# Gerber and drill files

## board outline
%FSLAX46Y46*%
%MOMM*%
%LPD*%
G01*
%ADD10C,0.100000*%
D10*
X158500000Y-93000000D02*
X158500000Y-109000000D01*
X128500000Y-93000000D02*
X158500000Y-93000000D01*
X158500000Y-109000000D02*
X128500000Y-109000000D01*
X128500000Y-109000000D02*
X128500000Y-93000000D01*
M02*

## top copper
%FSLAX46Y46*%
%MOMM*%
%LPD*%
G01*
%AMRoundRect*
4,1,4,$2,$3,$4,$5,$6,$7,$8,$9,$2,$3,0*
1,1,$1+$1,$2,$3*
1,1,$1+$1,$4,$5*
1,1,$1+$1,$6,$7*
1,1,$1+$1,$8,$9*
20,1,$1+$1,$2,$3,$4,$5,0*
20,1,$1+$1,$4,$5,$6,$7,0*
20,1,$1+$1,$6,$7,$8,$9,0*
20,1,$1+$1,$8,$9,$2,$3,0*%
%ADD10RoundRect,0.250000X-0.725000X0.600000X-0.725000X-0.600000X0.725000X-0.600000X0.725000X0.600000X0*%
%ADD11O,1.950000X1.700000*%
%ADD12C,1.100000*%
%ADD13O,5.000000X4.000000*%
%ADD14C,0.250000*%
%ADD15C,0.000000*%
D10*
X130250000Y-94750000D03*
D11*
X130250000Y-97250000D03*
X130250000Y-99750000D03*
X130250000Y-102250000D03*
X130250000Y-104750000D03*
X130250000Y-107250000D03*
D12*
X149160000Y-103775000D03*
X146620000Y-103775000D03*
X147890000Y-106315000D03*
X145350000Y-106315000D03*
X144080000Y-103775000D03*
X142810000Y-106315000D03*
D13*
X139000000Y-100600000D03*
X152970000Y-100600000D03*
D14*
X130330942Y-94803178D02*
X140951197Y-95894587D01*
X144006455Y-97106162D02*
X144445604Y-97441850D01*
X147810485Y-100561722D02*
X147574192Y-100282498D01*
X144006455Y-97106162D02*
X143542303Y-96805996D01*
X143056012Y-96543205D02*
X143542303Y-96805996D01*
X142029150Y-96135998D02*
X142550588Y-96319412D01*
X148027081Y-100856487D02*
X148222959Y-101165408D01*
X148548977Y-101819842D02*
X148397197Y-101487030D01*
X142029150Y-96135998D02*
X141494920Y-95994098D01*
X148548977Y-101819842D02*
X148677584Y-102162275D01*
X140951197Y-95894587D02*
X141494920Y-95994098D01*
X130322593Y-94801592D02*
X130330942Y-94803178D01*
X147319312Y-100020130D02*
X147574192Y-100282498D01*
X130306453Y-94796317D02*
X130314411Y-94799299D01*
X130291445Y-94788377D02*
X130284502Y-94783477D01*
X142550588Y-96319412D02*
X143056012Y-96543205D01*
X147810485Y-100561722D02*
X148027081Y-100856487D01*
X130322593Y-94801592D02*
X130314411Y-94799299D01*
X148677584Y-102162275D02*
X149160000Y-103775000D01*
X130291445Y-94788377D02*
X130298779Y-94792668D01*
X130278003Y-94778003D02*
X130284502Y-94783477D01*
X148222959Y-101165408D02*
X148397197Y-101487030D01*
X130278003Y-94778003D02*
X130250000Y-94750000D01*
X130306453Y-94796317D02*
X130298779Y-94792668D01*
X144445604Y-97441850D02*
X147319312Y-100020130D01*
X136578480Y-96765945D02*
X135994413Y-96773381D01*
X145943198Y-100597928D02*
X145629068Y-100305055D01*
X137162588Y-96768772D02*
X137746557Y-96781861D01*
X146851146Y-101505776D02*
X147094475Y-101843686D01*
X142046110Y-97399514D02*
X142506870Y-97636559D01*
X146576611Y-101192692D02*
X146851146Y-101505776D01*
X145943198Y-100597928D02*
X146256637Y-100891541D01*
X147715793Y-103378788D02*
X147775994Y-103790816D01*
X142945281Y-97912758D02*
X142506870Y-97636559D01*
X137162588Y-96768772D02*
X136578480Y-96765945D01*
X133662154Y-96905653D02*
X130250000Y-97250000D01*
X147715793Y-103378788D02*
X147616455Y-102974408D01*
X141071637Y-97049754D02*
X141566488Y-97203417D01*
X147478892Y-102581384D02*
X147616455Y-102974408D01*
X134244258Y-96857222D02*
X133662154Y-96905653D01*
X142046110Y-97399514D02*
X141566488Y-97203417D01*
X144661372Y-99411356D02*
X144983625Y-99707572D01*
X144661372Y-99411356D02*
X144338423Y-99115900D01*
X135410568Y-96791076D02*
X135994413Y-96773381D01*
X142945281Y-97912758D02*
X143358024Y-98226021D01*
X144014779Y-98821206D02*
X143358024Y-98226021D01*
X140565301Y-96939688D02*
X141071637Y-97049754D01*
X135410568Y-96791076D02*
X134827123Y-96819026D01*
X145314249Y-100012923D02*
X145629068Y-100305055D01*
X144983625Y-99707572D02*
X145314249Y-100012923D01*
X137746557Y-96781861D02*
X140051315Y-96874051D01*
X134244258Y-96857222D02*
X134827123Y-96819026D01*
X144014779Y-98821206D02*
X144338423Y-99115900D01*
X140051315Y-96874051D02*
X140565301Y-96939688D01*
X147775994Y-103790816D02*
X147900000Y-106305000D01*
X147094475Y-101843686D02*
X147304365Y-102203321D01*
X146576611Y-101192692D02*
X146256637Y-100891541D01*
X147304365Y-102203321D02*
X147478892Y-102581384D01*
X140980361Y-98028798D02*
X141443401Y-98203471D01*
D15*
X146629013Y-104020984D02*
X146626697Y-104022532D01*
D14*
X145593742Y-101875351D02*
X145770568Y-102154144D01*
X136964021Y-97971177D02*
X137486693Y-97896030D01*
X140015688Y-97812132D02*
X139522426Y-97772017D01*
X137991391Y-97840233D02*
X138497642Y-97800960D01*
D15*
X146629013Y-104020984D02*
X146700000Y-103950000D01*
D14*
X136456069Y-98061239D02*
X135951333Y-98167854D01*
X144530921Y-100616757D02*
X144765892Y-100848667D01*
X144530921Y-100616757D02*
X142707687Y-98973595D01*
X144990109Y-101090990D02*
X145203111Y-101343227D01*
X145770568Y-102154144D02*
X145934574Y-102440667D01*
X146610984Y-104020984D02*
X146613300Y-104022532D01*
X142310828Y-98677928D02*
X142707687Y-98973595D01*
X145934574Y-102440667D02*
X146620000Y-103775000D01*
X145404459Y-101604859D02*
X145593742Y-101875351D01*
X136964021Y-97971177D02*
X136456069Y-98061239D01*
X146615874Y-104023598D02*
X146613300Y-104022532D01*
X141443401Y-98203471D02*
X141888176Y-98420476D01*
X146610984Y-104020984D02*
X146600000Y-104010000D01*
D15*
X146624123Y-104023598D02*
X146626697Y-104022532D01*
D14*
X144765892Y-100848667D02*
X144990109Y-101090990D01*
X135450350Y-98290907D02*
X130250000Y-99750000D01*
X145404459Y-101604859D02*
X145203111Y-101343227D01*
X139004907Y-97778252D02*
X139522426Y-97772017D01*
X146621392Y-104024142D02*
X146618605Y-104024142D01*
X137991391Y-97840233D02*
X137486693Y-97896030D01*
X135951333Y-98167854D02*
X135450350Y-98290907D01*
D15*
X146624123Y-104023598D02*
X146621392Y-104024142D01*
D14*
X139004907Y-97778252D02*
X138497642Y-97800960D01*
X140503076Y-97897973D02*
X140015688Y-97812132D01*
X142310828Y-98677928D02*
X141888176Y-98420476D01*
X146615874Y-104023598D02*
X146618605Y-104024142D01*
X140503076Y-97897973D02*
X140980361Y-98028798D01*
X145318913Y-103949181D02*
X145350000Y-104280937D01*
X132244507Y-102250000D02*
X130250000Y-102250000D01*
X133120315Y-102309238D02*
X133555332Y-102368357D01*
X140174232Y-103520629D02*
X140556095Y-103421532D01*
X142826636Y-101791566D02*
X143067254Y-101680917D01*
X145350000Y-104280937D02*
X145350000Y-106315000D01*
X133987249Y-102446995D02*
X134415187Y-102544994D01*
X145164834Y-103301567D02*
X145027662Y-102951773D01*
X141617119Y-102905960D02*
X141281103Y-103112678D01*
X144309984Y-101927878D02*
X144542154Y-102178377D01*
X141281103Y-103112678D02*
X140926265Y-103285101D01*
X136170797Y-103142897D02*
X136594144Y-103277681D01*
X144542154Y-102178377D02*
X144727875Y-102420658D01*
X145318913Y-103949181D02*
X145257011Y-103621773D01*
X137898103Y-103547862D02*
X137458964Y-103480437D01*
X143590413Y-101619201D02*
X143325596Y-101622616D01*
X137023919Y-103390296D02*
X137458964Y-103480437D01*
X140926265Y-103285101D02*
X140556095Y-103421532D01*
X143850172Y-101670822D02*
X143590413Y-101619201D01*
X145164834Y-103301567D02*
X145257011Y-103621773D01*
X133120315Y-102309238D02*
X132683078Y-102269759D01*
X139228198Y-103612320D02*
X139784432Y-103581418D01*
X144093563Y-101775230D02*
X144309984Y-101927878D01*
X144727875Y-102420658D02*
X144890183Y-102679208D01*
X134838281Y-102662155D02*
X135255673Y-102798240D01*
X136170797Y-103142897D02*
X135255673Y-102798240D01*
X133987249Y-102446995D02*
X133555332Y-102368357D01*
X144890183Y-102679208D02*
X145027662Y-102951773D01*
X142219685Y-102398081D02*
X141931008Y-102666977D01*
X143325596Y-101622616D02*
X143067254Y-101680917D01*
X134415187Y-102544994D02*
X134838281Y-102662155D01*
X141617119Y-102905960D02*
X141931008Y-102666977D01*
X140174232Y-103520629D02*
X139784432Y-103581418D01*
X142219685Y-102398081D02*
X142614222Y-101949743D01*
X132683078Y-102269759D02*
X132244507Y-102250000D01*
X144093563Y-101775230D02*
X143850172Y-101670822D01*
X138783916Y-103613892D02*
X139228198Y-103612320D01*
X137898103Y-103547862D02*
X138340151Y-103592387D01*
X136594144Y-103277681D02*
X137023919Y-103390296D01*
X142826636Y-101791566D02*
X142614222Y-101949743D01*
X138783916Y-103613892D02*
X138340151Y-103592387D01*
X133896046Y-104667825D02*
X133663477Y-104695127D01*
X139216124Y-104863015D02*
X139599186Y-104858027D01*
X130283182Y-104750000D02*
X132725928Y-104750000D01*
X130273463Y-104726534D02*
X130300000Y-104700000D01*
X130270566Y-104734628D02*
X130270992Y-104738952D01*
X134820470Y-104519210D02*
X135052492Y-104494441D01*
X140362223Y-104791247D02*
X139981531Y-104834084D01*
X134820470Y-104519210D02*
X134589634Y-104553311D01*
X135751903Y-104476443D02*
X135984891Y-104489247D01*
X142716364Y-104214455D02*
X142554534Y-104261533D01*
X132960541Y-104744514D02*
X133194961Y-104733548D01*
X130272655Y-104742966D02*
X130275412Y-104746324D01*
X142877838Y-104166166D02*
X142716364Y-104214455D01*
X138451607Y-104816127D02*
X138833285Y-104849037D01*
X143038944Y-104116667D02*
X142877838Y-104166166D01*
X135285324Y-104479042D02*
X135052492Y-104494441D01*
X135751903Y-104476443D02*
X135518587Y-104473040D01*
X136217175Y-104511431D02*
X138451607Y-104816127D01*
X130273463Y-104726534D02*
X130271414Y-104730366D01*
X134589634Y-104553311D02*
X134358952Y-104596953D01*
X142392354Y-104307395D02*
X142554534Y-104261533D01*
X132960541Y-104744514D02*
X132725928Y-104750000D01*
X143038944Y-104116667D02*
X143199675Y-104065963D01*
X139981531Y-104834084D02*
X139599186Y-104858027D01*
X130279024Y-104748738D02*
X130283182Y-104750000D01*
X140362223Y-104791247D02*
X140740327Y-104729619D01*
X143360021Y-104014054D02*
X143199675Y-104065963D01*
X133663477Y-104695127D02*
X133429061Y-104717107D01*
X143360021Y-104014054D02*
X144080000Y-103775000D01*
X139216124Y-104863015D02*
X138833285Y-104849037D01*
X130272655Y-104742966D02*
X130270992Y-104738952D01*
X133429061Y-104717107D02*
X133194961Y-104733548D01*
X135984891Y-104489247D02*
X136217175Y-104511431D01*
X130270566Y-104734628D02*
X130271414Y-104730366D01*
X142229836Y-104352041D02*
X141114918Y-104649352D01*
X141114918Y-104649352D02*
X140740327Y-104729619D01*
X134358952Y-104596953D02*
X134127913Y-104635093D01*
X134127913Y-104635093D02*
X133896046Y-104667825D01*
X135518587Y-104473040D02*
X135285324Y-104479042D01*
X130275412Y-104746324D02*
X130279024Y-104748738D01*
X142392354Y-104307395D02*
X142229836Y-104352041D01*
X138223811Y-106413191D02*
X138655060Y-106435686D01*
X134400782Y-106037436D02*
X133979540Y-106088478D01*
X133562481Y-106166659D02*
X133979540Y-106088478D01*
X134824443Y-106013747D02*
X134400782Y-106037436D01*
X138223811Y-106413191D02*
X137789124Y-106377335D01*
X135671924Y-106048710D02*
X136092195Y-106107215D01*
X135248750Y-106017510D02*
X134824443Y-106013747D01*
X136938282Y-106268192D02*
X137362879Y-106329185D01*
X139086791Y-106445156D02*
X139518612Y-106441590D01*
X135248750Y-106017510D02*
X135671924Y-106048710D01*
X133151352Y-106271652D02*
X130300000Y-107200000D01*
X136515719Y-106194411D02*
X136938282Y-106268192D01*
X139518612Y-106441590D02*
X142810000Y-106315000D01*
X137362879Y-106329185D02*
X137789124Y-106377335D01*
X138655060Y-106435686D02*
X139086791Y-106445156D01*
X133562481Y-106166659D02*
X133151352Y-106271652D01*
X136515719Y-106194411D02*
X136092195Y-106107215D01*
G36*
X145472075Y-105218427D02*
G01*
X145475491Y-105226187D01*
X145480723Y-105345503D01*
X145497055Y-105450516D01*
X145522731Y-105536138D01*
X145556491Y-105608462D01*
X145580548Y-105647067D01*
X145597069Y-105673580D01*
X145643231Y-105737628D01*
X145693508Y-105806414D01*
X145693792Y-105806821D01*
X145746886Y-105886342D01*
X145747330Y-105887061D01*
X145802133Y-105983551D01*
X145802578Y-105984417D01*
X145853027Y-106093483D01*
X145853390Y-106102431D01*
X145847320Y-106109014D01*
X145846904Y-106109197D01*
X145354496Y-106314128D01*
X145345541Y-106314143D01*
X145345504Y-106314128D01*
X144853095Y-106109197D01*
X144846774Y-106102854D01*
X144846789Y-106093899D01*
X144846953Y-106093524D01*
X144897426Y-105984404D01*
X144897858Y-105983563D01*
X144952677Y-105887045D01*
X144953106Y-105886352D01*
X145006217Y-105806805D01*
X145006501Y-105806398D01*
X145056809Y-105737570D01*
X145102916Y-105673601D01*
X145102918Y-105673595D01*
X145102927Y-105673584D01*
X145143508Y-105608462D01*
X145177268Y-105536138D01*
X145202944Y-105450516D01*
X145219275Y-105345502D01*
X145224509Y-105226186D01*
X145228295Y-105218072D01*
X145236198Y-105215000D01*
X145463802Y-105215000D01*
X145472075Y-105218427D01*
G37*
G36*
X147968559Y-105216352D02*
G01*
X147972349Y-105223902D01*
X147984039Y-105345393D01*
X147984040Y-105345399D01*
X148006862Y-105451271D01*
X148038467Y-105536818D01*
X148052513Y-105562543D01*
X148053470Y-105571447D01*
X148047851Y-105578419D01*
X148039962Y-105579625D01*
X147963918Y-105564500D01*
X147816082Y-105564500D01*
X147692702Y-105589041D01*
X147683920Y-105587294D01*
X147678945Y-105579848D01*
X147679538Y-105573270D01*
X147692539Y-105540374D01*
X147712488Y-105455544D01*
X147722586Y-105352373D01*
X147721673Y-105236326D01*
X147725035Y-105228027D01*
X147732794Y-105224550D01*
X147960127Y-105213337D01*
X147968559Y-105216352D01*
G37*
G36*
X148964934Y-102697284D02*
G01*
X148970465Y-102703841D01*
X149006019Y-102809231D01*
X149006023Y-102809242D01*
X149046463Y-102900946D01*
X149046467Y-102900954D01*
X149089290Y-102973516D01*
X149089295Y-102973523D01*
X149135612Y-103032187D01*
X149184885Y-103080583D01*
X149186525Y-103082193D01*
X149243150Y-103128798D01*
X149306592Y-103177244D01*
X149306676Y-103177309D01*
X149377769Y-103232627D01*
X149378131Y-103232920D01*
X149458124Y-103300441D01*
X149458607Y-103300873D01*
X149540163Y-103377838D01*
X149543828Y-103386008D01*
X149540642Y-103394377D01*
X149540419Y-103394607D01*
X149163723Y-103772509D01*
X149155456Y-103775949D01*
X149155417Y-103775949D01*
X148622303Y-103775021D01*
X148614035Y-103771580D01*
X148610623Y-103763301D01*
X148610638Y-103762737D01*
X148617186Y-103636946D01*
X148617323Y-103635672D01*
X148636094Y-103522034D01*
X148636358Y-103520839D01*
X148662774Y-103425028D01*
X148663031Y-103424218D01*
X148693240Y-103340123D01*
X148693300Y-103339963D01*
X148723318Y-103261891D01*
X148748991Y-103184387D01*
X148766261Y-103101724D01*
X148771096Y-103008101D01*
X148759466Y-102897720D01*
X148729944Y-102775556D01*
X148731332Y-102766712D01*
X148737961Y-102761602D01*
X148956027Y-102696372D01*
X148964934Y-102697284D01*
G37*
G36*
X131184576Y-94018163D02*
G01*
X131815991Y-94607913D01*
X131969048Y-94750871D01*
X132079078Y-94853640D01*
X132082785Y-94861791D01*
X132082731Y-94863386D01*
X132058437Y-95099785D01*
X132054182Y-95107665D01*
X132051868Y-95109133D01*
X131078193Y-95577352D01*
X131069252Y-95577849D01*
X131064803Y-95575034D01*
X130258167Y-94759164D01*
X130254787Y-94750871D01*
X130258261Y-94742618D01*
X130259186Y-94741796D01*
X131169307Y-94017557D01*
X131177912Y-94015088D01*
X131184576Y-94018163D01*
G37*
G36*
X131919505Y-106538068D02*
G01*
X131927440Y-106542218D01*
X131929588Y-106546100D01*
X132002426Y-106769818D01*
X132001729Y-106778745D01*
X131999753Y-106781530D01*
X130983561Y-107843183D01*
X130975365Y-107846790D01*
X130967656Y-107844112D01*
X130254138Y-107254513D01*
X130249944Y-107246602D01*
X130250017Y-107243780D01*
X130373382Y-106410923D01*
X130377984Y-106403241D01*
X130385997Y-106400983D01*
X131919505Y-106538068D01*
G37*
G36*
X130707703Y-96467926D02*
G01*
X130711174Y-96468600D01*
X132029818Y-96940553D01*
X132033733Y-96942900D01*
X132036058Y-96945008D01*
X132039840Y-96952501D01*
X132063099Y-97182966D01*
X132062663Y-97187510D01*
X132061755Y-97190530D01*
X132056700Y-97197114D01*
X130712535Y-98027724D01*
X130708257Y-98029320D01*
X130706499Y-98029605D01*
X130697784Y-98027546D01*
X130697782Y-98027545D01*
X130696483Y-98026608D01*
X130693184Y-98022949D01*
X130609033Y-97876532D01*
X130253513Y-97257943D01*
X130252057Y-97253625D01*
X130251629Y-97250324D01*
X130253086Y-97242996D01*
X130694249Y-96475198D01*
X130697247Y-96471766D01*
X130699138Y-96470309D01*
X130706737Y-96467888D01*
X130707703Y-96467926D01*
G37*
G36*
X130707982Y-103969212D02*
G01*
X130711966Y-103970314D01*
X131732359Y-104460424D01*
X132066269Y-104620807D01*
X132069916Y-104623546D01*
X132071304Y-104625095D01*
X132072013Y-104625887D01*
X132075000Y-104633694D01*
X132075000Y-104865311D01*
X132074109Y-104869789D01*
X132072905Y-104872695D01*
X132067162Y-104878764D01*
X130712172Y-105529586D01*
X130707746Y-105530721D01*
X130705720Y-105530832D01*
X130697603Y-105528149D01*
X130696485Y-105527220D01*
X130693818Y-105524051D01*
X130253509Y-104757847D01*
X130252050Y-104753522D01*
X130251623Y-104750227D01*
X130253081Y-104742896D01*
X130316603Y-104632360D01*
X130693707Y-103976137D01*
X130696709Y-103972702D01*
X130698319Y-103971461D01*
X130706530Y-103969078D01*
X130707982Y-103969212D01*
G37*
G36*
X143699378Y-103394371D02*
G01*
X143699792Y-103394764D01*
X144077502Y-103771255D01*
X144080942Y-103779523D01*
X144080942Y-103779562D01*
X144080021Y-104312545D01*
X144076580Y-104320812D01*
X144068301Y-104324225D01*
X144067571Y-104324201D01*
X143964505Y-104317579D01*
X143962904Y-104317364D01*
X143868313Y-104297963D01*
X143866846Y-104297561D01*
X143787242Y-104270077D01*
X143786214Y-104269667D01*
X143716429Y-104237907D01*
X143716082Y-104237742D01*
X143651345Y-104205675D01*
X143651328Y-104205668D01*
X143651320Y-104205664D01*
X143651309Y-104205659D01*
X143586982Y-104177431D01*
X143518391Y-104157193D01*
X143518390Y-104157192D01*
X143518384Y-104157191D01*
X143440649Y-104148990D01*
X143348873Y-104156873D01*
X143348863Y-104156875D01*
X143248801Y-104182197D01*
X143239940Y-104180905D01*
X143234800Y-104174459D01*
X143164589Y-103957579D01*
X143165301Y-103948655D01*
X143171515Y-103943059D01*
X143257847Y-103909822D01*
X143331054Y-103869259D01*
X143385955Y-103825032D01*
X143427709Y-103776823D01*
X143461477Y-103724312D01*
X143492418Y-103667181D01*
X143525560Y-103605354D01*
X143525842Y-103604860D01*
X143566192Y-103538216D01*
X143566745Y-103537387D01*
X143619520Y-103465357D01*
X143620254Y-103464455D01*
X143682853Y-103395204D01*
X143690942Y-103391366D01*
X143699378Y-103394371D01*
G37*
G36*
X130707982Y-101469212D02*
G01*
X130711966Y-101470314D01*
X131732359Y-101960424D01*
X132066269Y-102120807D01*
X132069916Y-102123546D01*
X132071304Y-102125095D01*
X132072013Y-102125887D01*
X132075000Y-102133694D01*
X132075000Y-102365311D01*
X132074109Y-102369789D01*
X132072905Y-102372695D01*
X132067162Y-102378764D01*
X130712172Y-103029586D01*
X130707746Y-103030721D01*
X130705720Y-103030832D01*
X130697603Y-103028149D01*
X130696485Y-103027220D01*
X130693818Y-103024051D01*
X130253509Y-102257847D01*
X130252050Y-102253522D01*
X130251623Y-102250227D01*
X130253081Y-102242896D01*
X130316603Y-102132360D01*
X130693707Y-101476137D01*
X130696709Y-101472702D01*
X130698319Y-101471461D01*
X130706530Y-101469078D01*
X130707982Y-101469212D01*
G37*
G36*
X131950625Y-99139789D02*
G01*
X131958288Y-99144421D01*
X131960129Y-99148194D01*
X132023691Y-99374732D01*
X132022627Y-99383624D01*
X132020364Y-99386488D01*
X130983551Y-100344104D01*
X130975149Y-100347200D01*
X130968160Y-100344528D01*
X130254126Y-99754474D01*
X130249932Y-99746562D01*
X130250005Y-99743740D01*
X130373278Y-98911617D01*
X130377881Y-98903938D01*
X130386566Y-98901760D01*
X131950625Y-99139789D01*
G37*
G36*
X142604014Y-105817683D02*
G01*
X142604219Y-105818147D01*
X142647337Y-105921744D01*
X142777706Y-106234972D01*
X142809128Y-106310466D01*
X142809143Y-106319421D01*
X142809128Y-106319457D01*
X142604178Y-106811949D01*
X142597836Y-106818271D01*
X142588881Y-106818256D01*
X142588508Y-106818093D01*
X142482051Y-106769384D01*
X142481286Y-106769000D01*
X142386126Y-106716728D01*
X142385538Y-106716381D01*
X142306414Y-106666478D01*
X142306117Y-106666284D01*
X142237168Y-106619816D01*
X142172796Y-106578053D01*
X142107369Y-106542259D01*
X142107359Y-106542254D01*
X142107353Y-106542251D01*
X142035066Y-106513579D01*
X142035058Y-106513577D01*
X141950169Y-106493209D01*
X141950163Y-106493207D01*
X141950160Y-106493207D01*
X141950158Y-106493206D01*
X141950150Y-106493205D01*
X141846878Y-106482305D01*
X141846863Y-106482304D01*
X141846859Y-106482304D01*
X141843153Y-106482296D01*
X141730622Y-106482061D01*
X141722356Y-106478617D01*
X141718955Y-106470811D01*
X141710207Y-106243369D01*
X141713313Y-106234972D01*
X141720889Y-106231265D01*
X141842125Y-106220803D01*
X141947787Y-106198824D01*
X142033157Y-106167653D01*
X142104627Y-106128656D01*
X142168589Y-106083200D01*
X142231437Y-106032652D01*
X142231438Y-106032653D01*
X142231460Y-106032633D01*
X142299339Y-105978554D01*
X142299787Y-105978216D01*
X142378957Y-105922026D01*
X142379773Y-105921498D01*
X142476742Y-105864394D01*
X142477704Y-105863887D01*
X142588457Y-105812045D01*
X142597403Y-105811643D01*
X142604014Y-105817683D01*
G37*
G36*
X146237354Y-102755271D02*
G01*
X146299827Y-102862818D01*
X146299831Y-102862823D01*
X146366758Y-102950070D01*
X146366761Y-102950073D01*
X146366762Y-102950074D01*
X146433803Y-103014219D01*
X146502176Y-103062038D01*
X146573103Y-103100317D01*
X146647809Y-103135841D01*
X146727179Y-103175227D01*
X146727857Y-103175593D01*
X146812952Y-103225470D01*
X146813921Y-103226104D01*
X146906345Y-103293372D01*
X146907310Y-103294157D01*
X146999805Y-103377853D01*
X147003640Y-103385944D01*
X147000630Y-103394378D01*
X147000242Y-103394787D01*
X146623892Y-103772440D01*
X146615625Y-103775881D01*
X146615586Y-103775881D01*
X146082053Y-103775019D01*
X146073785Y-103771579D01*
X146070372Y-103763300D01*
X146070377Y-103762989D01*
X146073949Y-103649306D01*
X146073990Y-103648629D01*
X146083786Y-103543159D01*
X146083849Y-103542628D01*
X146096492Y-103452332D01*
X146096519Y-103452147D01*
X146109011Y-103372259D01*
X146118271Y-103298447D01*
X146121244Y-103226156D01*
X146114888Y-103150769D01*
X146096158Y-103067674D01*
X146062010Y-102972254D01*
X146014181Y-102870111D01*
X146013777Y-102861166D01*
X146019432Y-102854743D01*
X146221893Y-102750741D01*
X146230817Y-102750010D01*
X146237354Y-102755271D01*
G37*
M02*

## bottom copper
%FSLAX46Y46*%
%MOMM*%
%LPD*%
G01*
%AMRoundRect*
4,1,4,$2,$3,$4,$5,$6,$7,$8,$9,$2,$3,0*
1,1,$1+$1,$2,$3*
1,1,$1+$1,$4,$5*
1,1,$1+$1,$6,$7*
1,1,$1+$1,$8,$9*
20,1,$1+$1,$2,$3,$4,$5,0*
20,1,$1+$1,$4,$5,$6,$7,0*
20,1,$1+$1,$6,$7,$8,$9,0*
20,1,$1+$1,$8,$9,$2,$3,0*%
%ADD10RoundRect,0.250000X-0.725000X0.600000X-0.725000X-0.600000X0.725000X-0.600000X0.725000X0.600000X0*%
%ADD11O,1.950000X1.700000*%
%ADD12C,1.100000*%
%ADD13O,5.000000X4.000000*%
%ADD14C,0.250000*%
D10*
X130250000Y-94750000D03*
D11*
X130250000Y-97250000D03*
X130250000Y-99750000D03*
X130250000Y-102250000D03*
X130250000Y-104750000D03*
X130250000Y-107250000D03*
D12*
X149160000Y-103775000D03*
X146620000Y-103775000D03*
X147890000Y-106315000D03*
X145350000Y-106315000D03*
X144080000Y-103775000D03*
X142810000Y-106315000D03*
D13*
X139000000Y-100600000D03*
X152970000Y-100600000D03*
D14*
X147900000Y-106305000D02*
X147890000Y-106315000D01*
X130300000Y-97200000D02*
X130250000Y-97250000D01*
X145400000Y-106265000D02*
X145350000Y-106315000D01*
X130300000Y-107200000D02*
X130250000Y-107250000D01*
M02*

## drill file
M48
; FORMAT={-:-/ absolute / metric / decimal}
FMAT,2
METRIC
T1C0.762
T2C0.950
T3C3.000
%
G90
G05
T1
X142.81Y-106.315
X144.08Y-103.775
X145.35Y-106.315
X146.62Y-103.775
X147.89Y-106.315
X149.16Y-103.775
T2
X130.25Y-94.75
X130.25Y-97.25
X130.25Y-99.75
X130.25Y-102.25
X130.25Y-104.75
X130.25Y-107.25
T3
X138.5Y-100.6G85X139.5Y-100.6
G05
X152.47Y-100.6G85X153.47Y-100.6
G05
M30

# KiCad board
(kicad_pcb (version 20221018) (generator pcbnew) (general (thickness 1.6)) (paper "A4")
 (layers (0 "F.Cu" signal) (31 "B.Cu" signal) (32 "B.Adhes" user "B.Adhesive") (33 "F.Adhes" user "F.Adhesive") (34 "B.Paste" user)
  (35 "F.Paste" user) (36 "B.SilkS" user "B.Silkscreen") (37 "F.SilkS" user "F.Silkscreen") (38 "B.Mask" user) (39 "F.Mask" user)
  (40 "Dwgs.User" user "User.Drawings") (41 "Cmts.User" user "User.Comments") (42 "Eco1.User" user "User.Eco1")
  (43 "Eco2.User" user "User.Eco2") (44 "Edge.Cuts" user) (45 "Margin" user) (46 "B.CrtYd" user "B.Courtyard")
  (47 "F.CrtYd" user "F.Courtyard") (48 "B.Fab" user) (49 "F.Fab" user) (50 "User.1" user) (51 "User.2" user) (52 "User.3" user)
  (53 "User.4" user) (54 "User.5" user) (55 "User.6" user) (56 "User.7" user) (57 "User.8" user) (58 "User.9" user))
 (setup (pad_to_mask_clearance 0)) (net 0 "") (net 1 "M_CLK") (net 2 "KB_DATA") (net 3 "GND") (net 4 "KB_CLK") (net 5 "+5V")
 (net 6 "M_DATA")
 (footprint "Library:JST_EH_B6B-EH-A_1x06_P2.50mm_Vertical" (layer "F.Cu") (at 130.25 94.75 -90)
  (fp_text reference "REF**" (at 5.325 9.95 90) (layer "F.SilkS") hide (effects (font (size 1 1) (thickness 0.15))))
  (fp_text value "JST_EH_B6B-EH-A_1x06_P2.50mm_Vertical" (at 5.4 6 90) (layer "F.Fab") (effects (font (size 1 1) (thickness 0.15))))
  (pad "1" thru_hole roundrect (at 0 0 270) (size 1.7 1.95) (drill 0.95) (layers "*.Cu" "*.Mask") (roundrect_rratio 0.1470588235)
   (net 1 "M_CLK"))
  (pad "2" thru_hole oval (at 2.5 0 270) (size 1.7 1.95) (drill 0.95) (layers "*.Cu" "*.Mask") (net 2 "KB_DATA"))
  (pad "3" thru_hole oval (at 5 0 270) (size 1.7 1.95) (drill 0.95) (layers "*.Cu" "*.Mask") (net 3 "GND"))
  (pad "4" thru_hole oval (at 7.5 0 270) (size 1.7 1.95) (drill 0.95) (layers "*.Cu" "*.Mask") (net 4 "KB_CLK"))
  (pad "5" thru_hole oval (at 10 0 270) (size 1.7 1.95) (drill 0.95) (layers "*.Cu" "*.Mask") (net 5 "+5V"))
  (pad "6" thru_hole oval (at 12.5 0 270) (size 1.7 1.95) (drill 0.95) (layers "*.Cu" "*.Mask") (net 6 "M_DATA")))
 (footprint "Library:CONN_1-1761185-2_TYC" (layer "F.Cu") (at 142.81 106.315)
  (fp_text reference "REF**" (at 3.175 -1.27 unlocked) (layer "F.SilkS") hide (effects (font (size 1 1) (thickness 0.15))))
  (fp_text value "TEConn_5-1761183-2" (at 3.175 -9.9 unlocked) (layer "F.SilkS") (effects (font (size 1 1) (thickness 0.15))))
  (pad "1" thru_hole circle (at 6.35 -2.54) (size 1.1 1.1) (drill 0.762) (layers "*.Cu" "*.Mask") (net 1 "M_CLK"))
  (pad "3" thru_hole circle (at 3.81 -2.54) (size 1.1 1.1) (drill 0.762) (layers "*.Cu" "*.Mask") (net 3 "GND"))
  (pad "3" thru_hole circle (at 5.08 0) (size 1.1 1.1) (drill 0.762) (layers "*.Cu" "*.Mask") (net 3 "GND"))
  (pad "4" thru_hole circle (at 2.54 0) (size 1.1 1.1) (drill 0.762) (layers "*.Cu" "*.Mask") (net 4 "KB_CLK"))
  (pad "5" thru_hole circle (at 1.27 -2.54) (size 1.1 1.1) (drill 0.762) (layers "*.Cu" "*.Mask") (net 5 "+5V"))
  (pad "6" thru_hole circle (at 0 0) (size 1.1 1.1) (drill 0.762) (layers "*.Cu" "*.Mask") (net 6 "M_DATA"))
  (pad "13" thru_hole oval (at -3.81 -5.715) (size 5 4) (drill oval 4 3) (layers "*.Cu" "*.Mask"))
  (pad "14" thru_hole oval (at 10.16 -5.715) (size 5 4) (drill oval 4 3) (layers "*.Cu" "*.Mask")))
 (gr_line (start 158.5 93) (end 158.5 109) (stroke (width 0.1) (type default)) (layer "Edge.Cuts"))
 (gr_line (start 128.5 93) (end 158.5 93) (stroke (width 0.1) (type default)) (layer "Edge.Cuts"))
 (gr_line (start 158.5 109) (end 128.5 109) (stroke (width 0.1) (type default)) (layer "Edge.Cuts"))
 (gr_line (start 128.5 109) (end 128.5 93) (stroke (width 0.1) (type default)) (layer "Edge.Cuts"))
 (segment (start 130.330942 94.803178) (end 140.951197 95.894587) (width 0.25) (layer "F.Cu") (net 1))
 (segment (start 144.006455 97.106162) (end 144.445604 97.44185) (width 0.25) (layer "F.Cu") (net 1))
 (segment (start 147.810485 100.561722) (end 147.574192 100.282498) (width 0.25) (layer "F.Cu") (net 1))
 (segment (start 144.006455 97.106162) (end 143.542303 96.805996) (width 0.25) (layer "F.Cu") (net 1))
 (segment (start 143.056012 96.543205) (end 143.542303 96.805996) (width 0.25) (layer "F.Cu") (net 1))
 (segment (start 142.02915 96.135998) (end 142.550588 96.319412) (width 0.25) (layer "F.Cu") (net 1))
 (segment (start 148.027081 100.856487) (end 148.222959 101.165408) (width 0.25) (layer "F.Cu") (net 1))
 (segment (start 148.548977 101.819842) (end 148.397197 101.48703) (width 0.25) (layer "F.Cu") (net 1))
 (segment (start 142.02915 96.135998) (end 141.49492 95.994098) (width 0.25) (layer "F.Cu") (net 1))
 (segment (start 148.548977 101.819842) (end 148.677584 102.162275) (width 0.25) (layer "F.Cu") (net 1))
 (segment (start 140.951197 95.894587) (end 141.49492 95.994098) (width 0.25) (layer "F.Cu") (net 1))
 (segment (start 130.322593 94.801592) (end 130.330942 94.803178) (width 0.25) (layer "F.Cu") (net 1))
 (segment (start 147.319312 100.02013) (end 147.574192 100.282498) (width 0.25) (layer "F.Cu") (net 1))
 (segment (start 130.306453 94.796317) (end 130.314411 94.799299) (width 0.25) (layer "F.Cu") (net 1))
 (segment (start 130.291445 94.788377) (end 130.284502 94.783477) (width 0.25) (layer "F.Cu") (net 1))
 (segment (start 142.550588 96.319412) (end 143.056012 96.543205) (width 0.25) (layer "F.Cu") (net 1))
 (segment (start 147.810485 100.561722) (end 148.027081 100.856487) (width 0.25) (layer "F.Cu") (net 1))
 (segment (start 130.322593 94.801592) (end 130.314411 94.799299) (width 0.25) (layer "F.Cu") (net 1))
 (segment (start 148.677584 102.162275) (end 149.16 103.775) (width 0.25) (layer "F.Cu") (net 1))
 (segment (start 130.291445 94.788377) (end 130.298779 94.792668) (width 0.25) (layer "F.Cu") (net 1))
 (segment (start 130.278003 94.778003) (end 130.284502 94.783477) (width 0.25) (layer "F.Cu") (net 1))
 (segment (start 148.222959 101.165408) (end 148.397197 101.48703) (width 0.25) (layer "F.Cu") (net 1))
 (segment (start 130.278003 94.778003) (end 130.25 94.75) (width 0.25) (layer "F.Cu") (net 1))
 (segment (start 130.306453 94.796317) (end 130.298779 94.792668) (width 0.25) (layer "F.Cu") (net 1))
 (segment (start 144.445604 97.44185) (end 147.319312 100.02013) (width 0.25) (layer "F.Cu") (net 1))
 (segment (start 136.57848 96.765945) (end 135.994413 96.773381) (width 0.25) (layer "F.Cu") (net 2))
 (segment (start 145.943198 100.597928) (end 145.629068 100.305055) (width 0.25) (layer "F.Cu") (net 2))
 (segment (start 137.162588 96.768772) (end 137.746557 96.781861) (width 0.25) (layer "F.Cu") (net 2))
 (segment (start 146.851146 101.505776) (end 147.094475 101.843686) (width 0.25) (layer "F.Cu") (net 2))
 (segment (start 142.04611 97.399514) (end 142.50687 97.636559) (width 0.25) (layer "F.Cu") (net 2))
 (segment (start 146.576611 101.192692) (end 146.851146 101.505776) (width 0.25) (layer "F.Cu") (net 2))
 (segment (start 145.943198 100.597928) (end 146.256637 100.891541) (width 0.25) (layer "F.Cu") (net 2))
 (segment (start 147.715793 103.378788) (end 147.775994 103.790816) (width 0.25) (layer "F.Cu") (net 2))
 (segment (start 142.945281 97.912758) (end 142.50687 97.636559) (width 0.25) (layer "F.Cu") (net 2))
 (segment (start 137.162588 96.768772) (end 136.57848 96.765945) (width 0.25) (layer "F.Cu") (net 2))
 (segment (start 133.662154 96.905653) (end 130.25 97.25) (width 0.25) (layer "F.Cu") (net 2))
 (segment (start 147.715793 103.378788) (end 147.616455 102.974408) (width 0.25) (layer "F.Cu") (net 2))
 (segment (start 141.071637 97.049754) (end 141.566488 97.203417) (width 0.25) (layer "F.Cu") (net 2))
 (segment (start 147.478892 102.581384) (end 147.616455 102.974408) (width 0.25) (layer "F.Cu") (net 2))
 (segment (start 134.244258 96.857222) (end 133.662154 96.905653) (width 0.25) (layer "F.Cu") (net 2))
 (segment (start 142.04611 97.399514) (end 141.566488 97.203417) (width 0.25) (layer "F.Cu") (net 2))
 (segment (start 144.661372 99.411356) (end 144.983625 99.707572) (width 0.25) (layer "F.Cu") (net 2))
 (segment (start 144.661372 99.411356) (end 144.338423 99.1159) (width 0.25) (layer "F.Cu") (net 2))
 (segment (start 135.410568 96.791076) (end 135.994413 96.773381) (width 0.25) (layer "F.Cu") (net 2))
 (segment (start 142.945281 97.912758) (end 143.358024 98.226021) (width 0.25) (layer "F.Cu") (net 2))
 (segment (start 144.014779 98.821206) (end 143.358024 98.226021) (width 0.25) (layer "F.Cu") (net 2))
 (segment (start 140.565301 96.939688) (end 141.071637 97.049754) (width 0.25) (layer "F.Cu") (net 2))
 (segment (start 135.410568 96.791076) (end 134.827123 96.819026) (width 0.25) (layer "F.Cu") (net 2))
 (segment (start 145.314249 100.012923) (end 145.629068 100.305055) (width 0.25) (layer "F.Cu") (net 2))
 (segment (start 144.983625 99.707572) (end 145.314249 100.012923) (width 0.25) (layer "F.Cu") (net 2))
 (segment (start 137.746557 96.781861) (end 140.051315 96.874051) (width 0.25) (layer "F.Cu") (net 2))
 (segment (start 134.244258 96.857222) (end 134.827123 96.819026) (width 0.25) (layer "F.Cu") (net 2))
 (segment (start 144.014779 98.821206) (end 144.338423 99.1159) (width 0.25) (layer "F.Cu") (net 2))
 (segment (start 140.051315 96.874051) (end 140.565301 96.939688) (width 0.25) (layer "F.Cu") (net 2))
 (segment (start 147.775994 103.790816) (end 147.9 106.305) (width 0.25) (layer "F.Cu") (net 2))
 (segment (start 147.094475 101.843686) (end 147.304365 102.203321) (width 0.25) (layer "F.Cu") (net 2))
 (segment (start 146.576611 101.192692) (end 146.256637 100.891541) (width 0.25) (layer "F.Cu") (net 2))
 (segment (start 147.304365 102.203321) (end 147.478892 102.581384) (width 0.25) (layer "F.Cu") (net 2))
 (segment (start 147.9 106.305) (end 147.89 106.315) (width 0.25) (layer "B.Cu") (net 2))
 (segment (start 130.3 97.2) (end 130.25 97.25) (width 0.25) (layer "B.Cu") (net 2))
 (segment (start 140.980361 98.028798) (end 141.443401 98.203471) (width 0.25) (layer "F.Cu") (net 3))
 (segment (start 146.629013 104.020984) (end 146.626697 104.022532) (width 0) (layer "F.Cu") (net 3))
 (segment (start 145.593742 101.875351) (end 145.770568 102.154144) (width 0.25) (layer "F.Cu") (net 3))
 (segment (start 136.964021 97.971177) (end 137.486693 97.89603) (width 0.25) (layer "F.Cu") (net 3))
 (segment (start 140.015688 97.812132) (end 139.522426 97.772017) (width 0.25) (layer "F.Cu") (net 3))
 (segment (start 137.991391 97.840233) (end 138.497642 97.80096) (width 0.25) (layer "F.Cu") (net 3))
 (segment (start 146.629013 104.020984) (end 146.7 103.95) (width 0) (layer "F.Cu") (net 3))
 (segment (start 136.456069 98.061239) (end 135.951333 98.167854) (width 0.25) (layer "F.Cu") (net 3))
 (segment (start 144.530921 100.616757) (end 144.765892 100.848667) (width 0.25) (layer "F.Cu") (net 3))
 (segment (start 144.530921 100.616757) (end 142.707687 98.973595) (width 0.25) (layer "F.Cu") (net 3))
 (segment (start 144.990109 101.09099) (end 145.203111 101.343227) (width 0.25) (layer "F.Cu") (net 3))
 (segment (start 145.770568 102.154144) (end 145.934574 102.440667) (width 0.25) (layer "F.Cu") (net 3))
 (segment (start 146.610984 104.020984) (end 146.6133 104.022532) (width 0.25) (layer "F.Cu") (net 3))
 (segment (start 142.310828 98.677928) (end 142.707687 98.973595) (width 0.25) (layer "F.Cu") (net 3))
 (segment (start 145.934574 102.440667) (end 146.62 103.775) (width 0.25) (layer "F.Cu") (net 3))
 (segment (start 145.404459 101.604859) (end 145.593742 101.875351) (width 0.25) (layer "F.Cu") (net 3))
 (segment (start 136.964021 97.971177) (end 136.456069 98.061239) (width 0.25) (layer "F.Cu") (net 3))
 (segment (start 146.615874 104.023598) (end 146.6133 104.022532) (width 0.25) (layer "F.Cu") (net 3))
 (segment (start 141.443401 98.203471) (end 141.888176 98.420476) (width 0.25) (layer "F.Cu") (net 3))
 (segment (start 146.610984 104.020984) (end 146.6 104.01) (width 0.25) (layer "F.Cu") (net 3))
 (segment (start 146.624123 104.023598) (end 146.626697 104.022532) (width 0) (layer "F.Cu") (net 3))
 (segment (start 144.765892 100.848667) (end 144.990109 101.09099) (width 0.25) (layer "F.Cu") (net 3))
 (segment (start 135.45035 98.290907) (end 130.25 99.75) (width 0.25) (layer "F.Cu") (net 3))
 (segment (start 145.404459 101.604859) (end 145.203111 101.343227) (width 0.25) (layer "F.Cu") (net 3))
 (segment (start 139.004907 97.778252) (end 139.522426 97.772017) (width 0.25) (layer "F.Cu") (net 3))
 (segment (start 146.621392 104.024142) (end 146.618605 104.024142) (width 0.25) (layer "F.Cu") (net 3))
 (segment (start 137.991391 97.840233) (end 137.486693 97.89603) (width 0.25) (layer "F.Cu") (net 3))
 (segment (start 135.951333 98.167854) (end 135.45035 98.290907) (width 0.25) (layer "F.Cu") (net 3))
 (segment (start 146.624123 104.023598) (end 146.621392 104.024142) (width 0) (layer "F.Cu") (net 3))
 (segment (start 139.004907 97.778252) (end 138.497642 97.80096) (width 0.25) (layer "F.Cu") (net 3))
 (segment (start 140.503076 97.897973) (end 140.015688 97.812132) (width 0.25) (layer "F.Cu") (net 3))
 (segment (start 142.310828 98.677928) (end 141.888176 98.420476) (width 0.25) (layer "F.Cu") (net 3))
 (segment (start 146.615874 104.023598) (end 146.618605 104.024142) (width 0.25) (layer "F.Cu") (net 3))
 (segment (start 140.503076 97.897973) (end 140.980361 98.028798) (width 0.25) (layer "F.Cu") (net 3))
 (segment (start 145.318913 103.949181) (end 145.35 104.280937) (width 0.25) (layer "F.Cu") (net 4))
 (segment (start 132.244507 102.25) (end 130.25 102.25) (width 0.25) (layer "F.Cu") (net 4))
 (segment (start 133.120315 102.309238) (end 133.555332 102.368357) (width 0.25) (layer "F.Cu") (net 4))
 (segment (start 140.174232 103.520629) (end 140.556095 103.421532) (width 0.25) (layer "F.Cu") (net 4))
 (segment (start 142.826636 101.791566) (end 143.067254 101.680917) (width 0.25) (layer "F.Cu") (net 4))
 (segment (start 145.35 104.280937) (end 145.35 106.315) (width 0.25) (layer "F.Cu") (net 4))
 (segment (start 133.987249 102.446995) (end 134.415187 102.544994) (width 0.25) (layer "F.Cu") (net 4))
 (segment (start 145.164834 103.301567) (end 145.027662 102.951773) (width 0.25) (layer "F.Cu") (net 4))
 (segment (start 141.617119 102.90596) (end 141.281103 103.112678) (width 0.25) (layer "F.Cu") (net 4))
 (segment (start 144.309984 101.927878) (end 144.542154 102.178377) (width 0.25) (layer "F.Cu") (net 4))
 (segment (start 141.281103 103.112678) (end 140.926265 103.285101) (width 0.25) (layer "F.Cu") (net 4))
 (segment (start 136.170797 103.142897) (end 136.594144 103.277681) (width 0.25) (layer "F.Cu") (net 4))
 (segment (start 144.542154 102.178377) (end 144.727875 102.420658) (width 0.25) (layer "F.Cu") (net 4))
 (segment (start 145.318913 103.949181) (end 145.257011 103.621773) (width 0.25) (layer "F.Cu") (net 4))
 (segment (start 137.898103 103.547862) (end 137.458964 103.480437) (width 0.25) (layer "F.Cu") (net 4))
 (segment (start 143.590413 101.619201) (end 143.325596 101.622616) (width 0.25) (layer "F.Cu") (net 4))
 (segment (start 137.023919 103.390296) (end 137.458964 103.480437) (width 0.25) (layer "F.Cu") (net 4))
 (segment (start 140.926265 103.285101) (end 140.556095 103.421532) (width 0.25) (layer "F.Cu") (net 4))
 (segment (start 143.850172 101.670822) (end 143.590413 101.619201) (width 0.25) (layer "F.Cu") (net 4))
 (segment (start 145.164834 103.301567) (end 145.257011 103.621773) (width 0.25) (layer "F.Cu") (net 4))
 (segment (start 133.120315 102.309238) (end 132.683078 102.269759) (width 0.25) (layer "F.Cu") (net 4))
 (segment (start 139.228198 103.61232) (end 139.784432 103.581418) (width 0.25) (layer "F.Cu") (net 4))
 (segment (start 144.093563 101.77523) (end 144.309984 101.927878) (width 0.25) (layer "F.Cu") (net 4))
 (segment (start 144.727875 102.420658) (end 144.890183 102.679208) (width 0.25) (layer "F.Cu") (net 4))
 (segment (start 134.838281 102.662155) (end 135.255673 102.79824) (width 0.25) (layer "F.Cu") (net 4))
 (segment (start 136.170797 103.142897) (end 135.255673 102.79824) (width 0.25) (layer "F.Cu") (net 4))
 (segment (start 133.987249 102.446995) (end 133.555332 102.368357) (width 0.25) (layer "F.Cu") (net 4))
 (segment (start 144.890183 102.679208) (end 145.027662 102.951773) (width 0.25) (layer "F.Cu") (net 4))
 (segment (start 142.219685 102.398081) (end 141.931008 102.666977) (width 0.25) (layer "F.Cu") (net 4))
 (segment (start 143.325596 101.622616) (end 143.067254 101.680917) (width 0.25) (layer "F.Cu") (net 4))
 (segment (start 134.415187 102.544994) (end 134.838281 102.662155) (width 0.25) (layer "F.Cu") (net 4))
 (segment (start 141.617119 102.90596) (end 141.931008 102.666977) (width 0.25) (layer "F.Cu") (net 4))
 (segment (start 140.174232 103.520629) (end 139.784432 103.581418) (width 0.25) (layer "F.Cu") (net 4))
 (segment (start 142.219685 102.398081) (end 142.614222 101.949743) (width 0.25) (layer "F.Cu") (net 4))
 (segment (start 132.683078 102.269759) (end 132.244507 102.25) (width 0.25) (layer "F.Cu") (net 4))
 (segment (start 144.093563 101.77523) (end 143.850172 101.670822) (width 0.25) (layer "F.Cu") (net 4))
 (segment (start 138.783916 103.613892) (end 139.228198 103.61232) (width 0.25) (layer "F.Cu") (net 4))
 (segment (start 137.898103 103.547862) (end 138.340151 103.592387) (width 0.25) (layer "F.Cu") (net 4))
 (segment (start 136.594144 103.277681) (end 137.023919 103.390296) (width 0.25) (layer "F.Cu") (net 4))
 (segment (start 142.826636 101.791566) (end 142.614222 101.949743) (width 0.25) (layer "F.Cu") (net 4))
 (segment (start 138.783916 103.613892) (end 138.340151 103.592387) (width 0.25) (layer "F.Cu") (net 4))
 (segment (start 145.4 106.265) (end 145.35 106.315) (width 0.25) (layer "B.Cu") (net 4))
 (segment (start 133.896046 104.667825) (end 133.663477 104.695127) (width 0.25) (layer "F.Cu") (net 5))
 (segment (start 139.216124 104.863015) (end 139.599186 104.858027) (width 0.25) (layer "F.Cu") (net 5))
 (segment (start 130.283182 104.75) (end 132.725928 104.75) (width 0.25) (layer "F.Cu") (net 5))
 (segment (start 130.273463 104.726534) (end 130.3 104.7) (width 0.25) (layer "F.Cu") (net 5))
 (segment (start 130.270566 104.734628) (end 130.270992 104.738952) (width 0.25) (layer "F.Cu") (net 5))
 (segment (start 134.82047 104.51921) (end 135.052492 104.494441) (width 0.25) (layer "F.Cu") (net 5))
 (segment (start 140.362223 104.791247) (end 139.981531 104.834084) (width 0.25) (layer "F.Cu") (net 5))
 (segment (start 134.82047 104.51921) (end 134.589634 104.553311) (width 0.25) (layer "F.Cu") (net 5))
 (segment (start 135.751903 104.476443) (end 135.984891 104.489247) (width 0.25) (layer "F.Cu") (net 5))
 (segment (start 142.716364 104.214455) (end 142.554534 104.261533) (width 0.25) (layer "F.Cu") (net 5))
 (segment (start 132.960541 104.744514) (end 133.194961 104.733548) (width 0.25) (layer "F.Cu") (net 5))
 (segment (start 130.272655 104.742966) (end 130.275412 104.746324) (width 0.25) (layer "F.Cu") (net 5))
 (segment (start 142.877838 104.166166) (end 142.716364 104.214455) (width 0.25) (layer "F.Cu") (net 5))
 (segment (start 138.451607 104.816127) (end 138.833285 104.849037) (width 0.25) (layer "F.Cu") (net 5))
 (segment (start 143.038944 104.116667) (end 142.877838 104.166166) (width 0.25) (layer "F.Cu") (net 5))
 (segment (start 135.285324 104.479042) (end 135.052492 104.494441) (width 0.25) (layer "F.Cu") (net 5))
 (segment (start 135.751903 104.476443) (end 135.518587 104.47304) (width 0.25) (layer "F.Cu") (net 5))
 (segment (start 136.217175 104.511431) (end 138.451607 104.816127) (width 0.25) (layer "F.Cu") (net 5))
 (segment (start 130.273463 104.726534) (end 130.271414 104.730366) (width 0.25) (layer "F.Cu") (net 5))
 (segment (start 134.589634 104.553311) (end 134.358952 104.596953) (width 0.25) (layer "F.Cu") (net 5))
 (segment (start 142.392354 104.307395) (end 142.554534 104.261533) (width 0.25) (layer "F.Cu") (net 5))
 (segment (start 132.960541 104.744514) (end 132.725928 104.75) (width 0.25) (layer "F.Cu") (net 5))
 (segment (start 143.038944 104.116667) (end 143.199675 104.065963) (width 0.25) (layer "F.Cu") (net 5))
 (segment (start 139.981531 104.834084) (end 139.599186 104.858027) (width 0.25) (layer "F.Cu") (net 5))
 (segment (start 130.279024 104.748738) (end 130.283182 104.75) (width 0.25) (layer "F.Cu") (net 5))
 (segment (start 140.362223 104.791247) (end 140.740327 104.729619) (width 0.25) (layer "F.Cu") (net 5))
 (segment (start 143.360021 104.014054) (end 143.199675 104.065963) (width 0.25) (layer "F.Cu") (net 5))
 (segment (start 133.663477 104.695127) (end 133.429061 104.717107) (width 0.25) (layer "F.Cu") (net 5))
 (segment (start 143.360021 104.014054) (end 144.08 103.775) (width 0.25) (layer "F.Cu") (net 5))
 (segment (start 139.216124 104.863015) (end 138.833285 104.849037) (width 0.25) (layer "F.Cu") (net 5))
 (segment (start 130.272655 104.742966) (end 130.270992 104.738952) (width 0.25) (layer "F.Cu") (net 5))
 (segment (start 133.429061 104.717107) (end 133.194961 104.733548) (width 0.25) (layer "F.Cu") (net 5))
 (segment (start 135.984891 104.489247) (end 136.217175 104.511431) (width 0.25) (layer "F.Cu") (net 5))
 (segment (start 130.270566 104.734628) (end 130.271414 104.730366) (width 0.25) (layer "F.Cu") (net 5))
 (segment (start 142.229836 104.352041) (end 141.114918 104.649352) (width 0.25) (layer "F.Cu") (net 5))
 (segment (start 141.114918 104.649352) (end 140.740327 104.729619) (width 0.25) (layer "F.Cu") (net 5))
 (segment (start 134.358952 104.596953) (end 134.127913 104.635093) (width 0.25) (layer "F.Cu") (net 5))
 (segment (start 134.127913 104.635093) (end 133.896046 104.667825) (width 0.25) (layer "F.Cu") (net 5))
 (segment (start 135.518587 104.47304) (end 135.285324 104.479042) (width 0.25) (layer "F.Cu") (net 5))
 (segment (start 130.275412 104.746324) (end 130.279024 104.748738) (width 0.25) (layer "F.Cu") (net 5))
 (segment (start 142.392354 104.307395) (end 142.229836 104.352041) (width 0.25) (layer "F.Cu") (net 5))
 (segment (start 138.223811 106.413191) (end 138.65506 106.435686) (width 0.25) (layer "F.Cu") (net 6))
 (segment (start 134.400782 106.037436) (end 133.97954 106.088478) (width 0.25) (layer "F.Cu") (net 6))
 (segment (start 133.562481 106.166659) (end 133.97954 106.088478) (width 0.25) (layer "F.Cu") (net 6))
 (segment (start 134.824443 106.013747) (end 134.400782 106.037436) (width 0.25) (layer "F.Cu") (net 6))
 (segment (start 138.223811 106.413191) (end 137.789124 106.377335) (width 0.25) (layer "F.Cu") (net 6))
 (segment (start 135.671924 106.04871) (end 136.092195 106.107215) (width 0.25) (layer "F.Cu") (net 6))
 (segment (start 135.24875 106.01751) (end 134.824443 106.013747) (width 0.25) (layer "F.Cu") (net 6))
 (segment (start 136.938282 106.268192) (end 137.362879 106.329185) (width 0.25) (layer "F.Cu") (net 6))
 (segment (start 139.086791 106.445156) (end 139.518612 106.44159) (width 0.25) (layer "F.Cu") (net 6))
 (segment (start 135.24875 106.01751) (end 135.671924 106.04871) (width 0.25) (layer "F.Cu") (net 6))
 (segment (start 133.151352 106.271652) (end 130.3 107.2) (width 0.25) (layer "F.Cu") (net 6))
 (segment (start 136.515719 106.194411) (end 136.938282 106.268192) (width 0.25) (layer "F.Cu") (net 6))
 (segment (start 139.518612 106.44159) (end 142.81 106.315) (width 0.25) (layer "F.Cu") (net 6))
 (segment (start 137.362879 106.329185) (end 137.789124 106.377335) (width 0.25) (layer "F.Cu") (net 6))
 (segment (start 138.65506 106.435686) (end 139.086791 106.445156) (width 0.25) (layer "F.Cu") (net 6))
 (segment (start 133.562481 106.166659) (end 133.151352 106.271652) (width 0.25) (layer "F.Cu") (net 6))
 (segment (start 136.515719 106.194411) (end 136.092195 106.107215) (width 0.25) (layer "F.Cu") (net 6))
 (segment (start 130.3 107.2) (end 130.25 107.25) (width 0.25) (layer "B.Cu") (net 6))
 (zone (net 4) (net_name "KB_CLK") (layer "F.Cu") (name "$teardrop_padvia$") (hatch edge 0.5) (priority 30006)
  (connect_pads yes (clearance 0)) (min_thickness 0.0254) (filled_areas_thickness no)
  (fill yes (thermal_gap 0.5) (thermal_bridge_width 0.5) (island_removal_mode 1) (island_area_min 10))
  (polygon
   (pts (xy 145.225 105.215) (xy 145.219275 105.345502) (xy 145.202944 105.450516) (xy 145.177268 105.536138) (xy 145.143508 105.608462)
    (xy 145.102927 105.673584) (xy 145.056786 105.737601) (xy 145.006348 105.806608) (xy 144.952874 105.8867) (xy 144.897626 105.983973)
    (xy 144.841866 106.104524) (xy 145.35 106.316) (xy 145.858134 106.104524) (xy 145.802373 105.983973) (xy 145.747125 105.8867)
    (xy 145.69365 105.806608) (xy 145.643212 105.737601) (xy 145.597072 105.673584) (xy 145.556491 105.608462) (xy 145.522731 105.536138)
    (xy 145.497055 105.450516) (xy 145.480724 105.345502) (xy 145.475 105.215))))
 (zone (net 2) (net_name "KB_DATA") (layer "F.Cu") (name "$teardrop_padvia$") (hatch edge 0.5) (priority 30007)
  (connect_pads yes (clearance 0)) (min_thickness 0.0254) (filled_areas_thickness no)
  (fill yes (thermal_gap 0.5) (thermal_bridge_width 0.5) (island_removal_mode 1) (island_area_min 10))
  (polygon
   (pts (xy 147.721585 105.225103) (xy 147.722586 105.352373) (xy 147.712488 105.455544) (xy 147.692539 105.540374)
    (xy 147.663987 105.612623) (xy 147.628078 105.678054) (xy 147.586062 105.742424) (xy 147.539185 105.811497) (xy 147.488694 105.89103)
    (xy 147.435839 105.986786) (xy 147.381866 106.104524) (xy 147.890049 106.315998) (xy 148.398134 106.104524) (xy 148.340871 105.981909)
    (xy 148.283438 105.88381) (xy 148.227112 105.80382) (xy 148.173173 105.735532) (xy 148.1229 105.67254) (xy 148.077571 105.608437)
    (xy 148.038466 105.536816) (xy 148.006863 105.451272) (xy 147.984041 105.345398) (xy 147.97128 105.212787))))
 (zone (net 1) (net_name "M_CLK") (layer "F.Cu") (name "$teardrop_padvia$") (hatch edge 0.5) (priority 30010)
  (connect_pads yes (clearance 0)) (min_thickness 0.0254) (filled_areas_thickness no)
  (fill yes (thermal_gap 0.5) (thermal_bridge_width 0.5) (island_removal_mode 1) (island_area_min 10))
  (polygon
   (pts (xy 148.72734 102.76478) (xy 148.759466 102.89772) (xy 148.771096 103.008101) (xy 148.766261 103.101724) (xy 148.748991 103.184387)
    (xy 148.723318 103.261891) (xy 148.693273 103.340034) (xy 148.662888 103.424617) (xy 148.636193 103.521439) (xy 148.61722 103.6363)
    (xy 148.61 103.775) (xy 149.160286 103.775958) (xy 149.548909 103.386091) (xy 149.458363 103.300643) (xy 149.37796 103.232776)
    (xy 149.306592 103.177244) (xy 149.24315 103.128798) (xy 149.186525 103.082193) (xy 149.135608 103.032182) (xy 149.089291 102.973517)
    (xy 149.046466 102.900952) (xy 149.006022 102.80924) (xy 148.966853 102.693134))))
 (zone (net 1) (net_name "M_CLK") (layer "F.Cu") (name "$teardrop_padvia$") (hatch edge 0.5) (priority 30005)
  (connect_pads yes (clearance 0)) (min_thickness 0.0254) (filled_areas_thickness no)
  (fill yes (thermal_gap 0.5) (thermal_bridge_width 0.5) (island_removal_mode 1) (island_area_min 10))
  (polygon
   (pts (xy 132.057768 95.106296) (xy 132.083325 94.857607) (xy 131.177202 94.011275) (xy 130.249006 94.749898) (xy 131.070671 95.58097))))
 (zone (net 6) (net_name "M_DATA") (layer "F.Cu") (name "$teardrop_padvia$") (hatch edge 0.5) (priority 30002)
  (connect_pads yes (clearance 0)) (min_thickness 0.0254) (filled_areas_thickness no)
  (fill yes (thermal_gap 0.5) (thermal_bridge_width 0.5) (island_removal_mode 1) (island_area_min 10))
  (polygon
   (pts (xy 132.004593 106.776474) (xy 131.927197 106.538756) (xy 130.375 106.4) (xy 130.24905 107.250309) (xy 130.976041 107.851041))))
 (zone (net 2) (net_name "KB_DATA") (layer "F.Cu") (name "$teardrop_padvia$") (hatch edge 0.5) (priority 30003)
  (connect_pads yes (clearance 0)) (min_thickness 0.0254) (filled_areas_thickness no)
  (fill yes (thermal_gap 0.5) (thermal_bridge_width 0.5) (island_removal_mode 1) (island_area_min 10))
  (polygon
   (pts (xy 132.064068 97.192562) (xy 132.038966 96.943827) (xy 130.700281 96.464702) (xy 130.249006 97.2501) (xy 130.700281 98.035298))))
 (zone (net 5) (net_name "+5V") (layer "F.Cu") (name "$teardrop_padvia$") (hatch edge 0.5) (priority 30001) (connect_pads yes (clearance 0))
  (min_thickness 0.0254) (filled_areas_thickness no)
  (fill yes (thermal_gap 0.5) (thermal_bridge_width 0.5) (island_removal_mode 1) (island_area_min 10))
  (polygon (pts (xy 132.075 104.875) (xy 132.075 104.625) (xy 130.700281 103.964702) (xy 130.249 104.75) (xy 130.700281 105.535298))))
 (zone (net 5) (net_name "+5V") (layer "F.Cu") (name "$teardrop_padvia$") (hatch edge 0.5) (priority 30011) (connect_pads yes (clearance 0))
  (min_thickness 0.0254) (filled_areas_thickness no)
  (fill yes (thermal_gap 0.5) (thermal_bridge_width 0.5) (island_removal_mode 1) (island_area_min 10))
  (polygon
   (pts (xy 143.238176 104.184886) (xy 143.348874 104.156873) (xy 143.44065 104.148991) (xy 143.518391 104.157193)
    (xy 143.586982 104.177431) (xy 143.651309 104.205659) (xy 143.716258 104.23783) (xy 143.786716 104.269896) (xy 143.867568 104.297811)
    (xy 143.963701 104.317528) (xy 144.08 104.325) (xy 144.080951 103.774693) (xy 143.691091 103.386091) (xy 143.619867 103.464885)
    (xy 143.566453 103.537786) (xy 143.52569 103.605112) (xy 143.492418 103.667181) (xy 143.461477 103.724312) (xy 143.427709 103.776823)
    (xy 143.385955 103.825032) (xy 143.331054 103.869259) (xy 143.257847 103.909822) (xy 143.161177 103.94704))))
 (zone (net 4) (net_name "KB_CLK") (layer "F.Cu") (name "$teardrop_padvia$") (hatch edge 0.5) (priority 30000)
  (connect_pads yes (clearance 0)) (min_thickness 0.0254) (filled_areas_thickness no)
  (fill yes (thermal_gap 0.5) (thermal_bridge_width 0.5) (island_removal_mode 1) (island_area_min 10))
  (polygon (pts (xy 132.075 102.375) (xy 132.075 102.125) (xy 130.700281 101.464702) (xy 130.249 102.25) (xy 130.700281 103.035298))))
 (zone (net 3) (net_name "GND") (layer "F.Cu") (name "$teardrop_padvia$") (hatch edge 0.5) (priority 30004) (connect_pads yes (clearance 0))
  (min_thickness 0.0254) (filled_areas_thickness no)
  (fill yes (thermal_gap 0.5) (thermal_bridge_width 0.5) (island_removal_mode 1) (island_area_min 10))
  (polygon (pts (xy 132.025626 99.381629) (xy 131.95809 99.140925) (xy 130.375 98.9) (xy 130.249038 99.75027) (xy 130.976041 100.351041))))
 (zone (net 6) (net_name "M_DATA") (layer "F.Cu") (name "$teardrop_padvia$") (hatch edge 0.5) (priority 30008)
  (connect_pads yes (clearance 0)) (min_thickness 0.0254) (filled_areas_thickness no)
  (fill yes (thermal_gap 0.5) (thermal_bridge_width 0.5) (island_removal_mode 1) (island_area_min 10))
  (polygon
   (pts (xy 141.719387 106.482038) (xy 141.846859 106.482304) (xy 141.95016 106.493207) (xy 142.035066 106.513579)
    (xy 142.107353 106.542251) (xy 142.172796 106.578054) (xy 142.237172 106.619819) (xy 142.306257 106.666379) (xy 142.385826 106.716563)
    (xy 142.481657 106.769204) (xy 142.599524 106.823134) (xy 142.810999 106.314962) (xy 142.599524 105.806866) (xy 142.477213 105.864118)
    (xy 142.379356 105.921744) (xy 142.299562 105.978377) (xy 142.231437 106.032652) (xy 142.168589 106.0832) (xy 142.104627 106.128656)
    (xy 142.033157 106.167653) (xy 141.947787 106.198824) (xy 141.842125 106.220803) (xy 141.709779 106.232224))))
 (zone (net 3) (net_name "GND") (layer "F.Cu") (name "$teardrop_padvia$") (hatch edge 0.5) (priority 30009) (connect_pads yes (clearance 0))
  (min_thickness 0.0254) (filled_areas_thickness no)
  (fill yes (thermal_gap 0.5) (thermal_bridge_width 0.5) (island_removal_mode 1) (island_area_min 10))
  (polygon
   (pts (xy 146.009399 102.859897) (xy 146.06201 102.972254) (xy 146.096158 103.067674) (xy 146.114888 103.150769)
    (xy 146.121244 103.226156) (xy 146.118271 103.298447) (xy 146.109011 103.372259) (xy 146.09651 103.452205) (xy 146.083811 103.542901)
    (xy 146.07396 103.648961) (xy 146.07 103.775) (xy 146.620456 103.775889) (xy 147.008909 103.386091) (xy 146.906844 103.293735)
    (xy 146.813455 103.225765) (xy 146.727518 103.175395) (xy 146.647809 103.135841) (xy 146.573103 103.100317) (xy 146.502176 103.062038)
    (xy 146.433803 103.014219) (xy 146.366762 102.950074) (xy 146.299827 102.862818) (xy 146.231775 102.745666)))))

